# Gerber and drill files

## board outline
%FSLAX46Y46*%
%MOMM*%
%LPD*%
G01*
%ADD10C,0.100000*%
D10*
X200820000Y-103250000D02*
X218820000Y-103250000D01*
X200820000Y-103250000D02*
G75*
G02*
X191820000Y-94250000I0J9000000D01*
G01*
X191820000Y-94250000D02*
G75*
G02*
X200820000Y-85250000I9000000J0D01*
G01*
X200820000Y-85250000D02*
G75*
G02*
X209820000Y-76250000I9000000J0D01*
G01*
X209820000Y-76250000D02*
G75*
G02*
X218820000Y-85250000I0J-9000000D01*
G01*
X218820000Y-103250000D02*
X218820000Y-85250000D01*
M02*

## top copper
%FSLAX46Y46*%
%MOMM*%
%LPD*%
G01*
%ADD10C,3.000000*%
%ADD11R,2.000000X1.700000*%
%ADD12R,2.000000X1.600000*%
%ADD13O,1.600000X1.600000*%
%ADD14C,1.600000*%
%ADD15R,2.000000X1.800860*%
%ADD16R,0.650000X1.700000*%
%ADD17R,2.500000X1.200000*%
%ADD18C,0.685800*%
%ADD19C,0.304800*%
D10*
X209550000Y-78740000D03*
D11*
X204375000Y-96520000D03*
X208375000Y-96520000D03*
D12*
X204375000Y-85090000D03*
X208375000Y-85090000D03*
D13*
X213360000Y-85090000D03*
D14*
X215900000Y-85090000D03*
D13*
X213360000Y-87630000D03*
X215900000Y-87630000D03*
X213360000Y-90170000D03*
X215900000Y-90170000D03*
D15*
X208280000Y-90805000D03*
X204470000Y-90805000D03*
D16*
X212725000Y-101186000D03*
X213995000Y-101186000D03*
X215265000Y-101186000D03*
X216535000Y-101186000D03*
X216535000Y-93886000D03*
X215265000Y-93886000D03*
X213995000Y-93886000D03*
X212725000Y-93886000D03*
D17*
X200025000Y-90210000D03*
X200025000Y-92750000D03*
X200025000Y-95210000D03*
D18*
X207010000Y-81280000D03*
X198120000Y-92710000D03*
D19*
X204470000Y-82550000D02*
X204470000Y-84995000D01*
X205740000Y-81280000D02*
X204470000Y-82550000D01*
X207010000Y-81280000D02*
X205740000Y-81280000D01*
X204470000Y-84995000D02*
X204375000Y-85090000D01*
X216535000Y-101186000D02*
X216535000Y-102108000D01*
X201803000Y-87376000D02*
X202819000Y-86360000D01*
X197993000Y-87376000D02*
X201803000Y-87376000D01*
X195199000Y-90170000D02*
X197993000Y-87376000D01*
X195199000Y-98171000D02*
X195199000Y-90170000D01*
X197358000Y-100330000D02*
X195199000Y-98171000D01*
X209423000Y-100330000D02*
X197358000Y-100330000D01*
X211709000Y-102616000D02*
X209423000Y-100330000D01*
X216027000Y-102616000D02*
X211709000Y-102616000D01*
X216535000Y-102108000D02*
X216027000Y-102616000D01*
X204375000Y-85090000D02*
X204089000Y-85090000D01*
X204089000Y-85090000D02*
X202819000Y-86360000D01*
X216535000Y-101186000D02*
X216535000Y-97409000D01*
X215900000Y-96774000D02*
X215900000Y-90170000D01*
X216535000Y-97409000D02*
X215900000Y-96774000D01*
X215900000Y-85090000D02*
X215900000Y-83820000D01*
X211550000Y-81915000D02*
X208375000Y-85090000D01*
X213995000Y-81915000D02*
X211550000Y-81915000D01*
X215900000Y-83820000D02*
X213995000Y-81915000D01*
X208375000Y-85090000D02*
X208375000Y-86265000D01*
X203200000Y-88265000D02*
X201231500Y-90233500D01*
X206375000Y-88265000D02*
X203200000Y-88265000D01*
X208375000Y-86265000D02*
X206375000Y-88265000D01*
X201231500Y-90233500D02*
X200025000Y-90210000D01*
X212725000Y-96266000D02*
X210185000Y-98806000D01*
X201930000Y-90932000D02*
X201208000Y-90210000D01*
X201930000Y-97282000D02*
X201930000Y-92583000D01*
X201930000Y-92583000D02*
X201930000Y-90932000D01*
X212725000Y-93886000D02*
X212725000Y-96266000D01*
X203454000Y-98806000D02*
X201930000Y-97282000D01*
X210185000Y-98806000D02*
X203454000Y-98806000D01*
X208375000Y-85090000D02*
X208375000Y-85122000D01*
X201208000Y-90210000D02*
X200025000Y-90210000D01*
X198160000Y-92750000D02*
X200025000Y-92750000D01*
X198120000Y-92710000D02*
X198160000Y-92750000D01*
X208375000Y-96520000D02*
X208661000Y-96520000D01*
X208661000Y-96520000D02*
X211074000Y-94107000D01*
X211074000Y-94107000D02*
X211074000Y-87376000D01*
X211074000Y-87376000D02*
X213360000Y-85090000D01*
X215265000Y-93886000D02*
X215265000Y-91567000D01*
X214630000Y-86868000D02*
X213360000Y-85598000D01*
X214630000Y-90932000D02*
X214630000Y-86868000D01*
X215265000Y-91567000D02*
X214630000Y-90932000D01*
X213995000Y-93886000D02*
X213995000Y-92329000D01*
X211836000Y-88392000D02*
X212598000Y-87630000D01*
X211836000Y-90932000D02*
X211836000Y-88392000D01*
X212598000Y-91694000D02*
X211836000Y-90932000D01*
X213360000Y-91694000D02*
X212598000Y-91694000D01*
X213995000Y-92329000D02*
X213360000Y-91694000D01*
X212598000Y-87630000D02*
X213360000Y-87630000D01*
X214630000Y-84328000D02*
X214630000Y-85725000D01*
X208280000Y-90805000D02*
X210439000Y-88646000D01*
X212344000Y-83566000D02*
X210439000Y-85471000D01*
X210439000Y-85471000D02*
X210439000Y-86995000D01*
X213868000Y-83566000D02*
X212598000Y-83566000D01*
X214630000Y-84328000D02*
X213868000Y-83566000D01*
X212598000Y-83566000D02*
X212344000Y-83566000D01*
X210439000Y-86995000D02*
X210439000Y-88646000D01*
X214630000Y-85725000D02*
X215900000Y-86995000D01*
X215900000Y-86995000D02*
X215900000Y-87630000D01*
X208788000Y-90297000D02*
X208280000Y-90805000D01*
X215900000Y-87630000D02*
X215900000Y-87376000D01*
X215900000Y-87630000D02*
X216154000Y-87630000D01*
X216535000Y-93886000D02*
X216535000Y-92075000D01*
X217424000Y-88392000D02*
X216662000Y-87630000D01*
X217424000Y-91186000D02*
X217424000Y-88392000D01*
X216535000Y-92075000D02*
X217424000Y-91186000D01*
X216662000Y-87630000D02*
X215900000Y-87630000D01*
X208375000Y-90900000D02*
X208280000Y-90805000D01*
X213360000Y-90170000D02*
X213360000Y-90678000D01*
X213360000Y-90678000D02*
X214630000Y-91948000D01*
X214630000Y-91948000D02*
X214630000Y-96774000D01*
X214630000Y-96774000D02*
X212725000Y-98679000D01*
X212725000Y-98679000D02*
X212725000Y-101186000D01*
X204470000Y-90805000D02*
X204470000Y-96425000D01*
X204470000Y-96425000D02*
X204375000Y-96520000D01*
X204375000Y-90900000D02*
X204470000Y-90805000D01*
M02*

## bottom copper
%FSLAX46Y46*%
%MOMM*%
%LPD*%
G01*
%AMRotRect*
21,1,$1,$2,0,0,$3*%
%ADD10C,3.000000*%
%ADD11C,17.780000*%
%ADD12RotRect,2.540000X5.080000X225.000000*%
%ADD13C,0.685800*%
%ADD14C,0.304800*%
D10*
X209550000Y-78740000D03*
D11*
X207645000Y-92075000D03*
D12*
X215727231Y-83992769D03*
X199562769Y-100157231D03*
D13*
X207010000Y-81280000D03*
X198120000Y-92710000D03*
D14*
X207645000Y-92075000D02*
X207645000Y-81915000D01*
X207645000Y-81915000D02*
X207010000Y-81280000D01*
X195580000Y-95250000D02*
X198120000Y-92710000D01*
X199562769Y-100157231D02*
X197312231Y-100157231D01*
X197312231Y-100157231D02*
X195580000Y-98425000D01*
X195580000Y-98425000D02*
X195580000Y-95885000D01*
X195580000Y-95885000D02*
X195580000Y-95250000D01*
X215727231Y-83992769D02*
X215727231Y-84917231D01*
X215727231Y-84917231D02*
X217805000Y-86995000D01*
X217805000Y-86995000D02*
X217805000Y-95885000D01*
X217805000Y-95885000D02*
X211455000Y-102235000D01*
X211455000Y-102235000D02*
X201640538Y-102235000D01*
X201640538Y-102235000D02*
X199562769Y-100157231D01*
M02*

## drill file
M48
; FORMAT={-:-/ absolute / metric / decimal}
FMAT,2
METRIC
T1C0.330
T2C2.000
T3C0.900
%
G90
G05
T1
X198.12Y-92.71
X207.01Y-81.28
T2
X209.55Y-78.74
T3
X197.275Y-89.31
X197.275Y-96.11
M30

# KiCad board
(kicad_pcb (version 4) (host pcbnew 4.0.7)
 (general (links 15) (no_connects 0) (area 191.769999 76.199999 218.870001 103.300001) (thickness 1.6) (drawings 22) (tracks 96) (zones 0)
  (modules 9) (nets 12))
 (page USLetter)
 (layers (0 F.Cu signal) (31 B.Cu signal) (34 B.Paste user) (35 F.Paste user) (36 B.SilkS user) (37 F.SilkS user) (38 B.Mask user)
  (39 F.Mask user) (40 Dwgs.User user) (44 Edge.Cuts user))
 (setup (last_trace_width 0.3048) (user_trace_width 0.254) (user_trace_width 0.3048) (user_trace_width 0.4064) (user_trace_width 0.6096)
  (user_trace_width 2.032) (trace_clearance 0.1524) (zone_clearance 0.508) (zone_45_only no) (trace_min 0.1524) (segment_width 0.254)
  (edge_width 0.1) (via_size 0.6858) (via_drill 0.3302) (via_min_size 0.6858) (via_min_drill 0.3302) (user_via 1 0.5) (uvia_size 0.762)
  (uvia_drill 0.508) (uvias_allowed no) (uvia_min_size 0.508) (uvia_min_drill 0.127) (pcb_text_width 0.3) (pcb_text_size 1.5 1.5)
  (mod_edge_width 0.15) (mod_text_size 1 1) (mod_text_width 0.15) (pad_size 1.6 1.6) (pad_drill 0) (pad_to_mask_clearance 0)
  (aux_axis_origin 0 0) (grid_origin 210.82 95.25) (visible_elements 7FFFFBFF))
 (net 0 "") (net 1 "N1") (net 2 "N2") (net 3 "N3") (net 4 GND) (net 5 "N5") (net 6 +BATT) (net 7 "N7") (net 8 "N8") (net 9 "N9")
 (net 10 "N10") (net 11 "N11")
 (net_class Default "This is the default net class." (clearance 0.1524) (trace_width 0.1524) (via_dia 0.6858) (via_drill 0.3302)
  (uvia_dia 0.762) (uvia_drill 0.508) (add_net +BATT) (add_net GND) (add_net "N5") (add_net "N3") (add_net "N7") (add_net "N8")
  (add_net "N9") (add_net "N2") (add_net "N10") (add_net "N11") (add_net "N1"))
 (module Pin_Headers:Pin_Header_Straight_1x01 (layer F.Cu) (at 209.55 78.74)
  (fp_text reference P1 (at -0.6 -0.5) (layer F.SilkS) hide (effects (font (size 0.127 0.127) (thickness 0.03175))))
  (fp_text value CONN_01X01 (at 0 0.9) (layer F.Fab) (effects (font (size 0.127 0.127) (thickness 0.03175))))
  (pad 1 thru_hole circle (at 0 0) (size 3 3) (drill 2) (layers *.Cu *.Mask) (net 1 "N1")))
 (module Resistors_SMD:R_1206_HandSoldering (layer F.Cu) (at 206.375 96.52)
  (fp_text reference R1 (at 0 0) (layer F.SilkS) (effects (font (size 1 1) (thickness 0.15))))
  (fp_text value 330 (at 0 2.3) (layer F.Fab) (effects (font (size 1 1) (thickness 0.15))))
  (pad 1 smd rect (at -2 0) (size 2 1.7) (layers F.Cu F.Paste F.Mask) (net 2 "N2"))
  (pad 2 smd rect (at 2 0) (size 2 1.7) (layers F.Cu F.Paste F.Mask) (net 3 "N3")))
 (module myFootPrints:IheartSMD (layer F.Cu) (at 203.835 100.33)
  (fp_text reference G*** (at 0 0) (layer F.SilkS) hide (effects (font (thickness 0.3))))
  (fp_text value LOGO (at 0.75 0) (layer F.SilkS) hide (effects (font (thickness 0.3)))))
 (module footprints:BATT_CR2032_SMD (layer B.Cu) (at 207.645 92.075 225)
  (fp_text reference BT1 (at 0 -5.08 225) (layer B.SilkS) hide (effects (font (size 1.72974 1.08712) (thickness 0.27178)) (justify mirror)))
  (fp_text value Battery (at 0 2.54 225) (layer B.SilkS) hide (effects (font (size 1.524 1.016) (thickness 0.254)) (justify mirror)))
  (pad 2 smd circle (at 0 0 225) (size 17.78 17.78) (layers B.Cu B.Paste B.Mask) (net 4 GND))
  (pad 1 smd rect (at -11.43 0 225) (size 2.54 5.08) (layers B.Cu B.Paste B.Mask) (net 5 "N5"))
  (pad 1 smd rect (at 11.43 0 225) (size 2.54 5.08) (layers B.Cu B.Paste B.Mask) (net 5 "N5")))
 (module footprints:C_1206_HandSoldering (layer F.Cu) (at 206.375 85.09)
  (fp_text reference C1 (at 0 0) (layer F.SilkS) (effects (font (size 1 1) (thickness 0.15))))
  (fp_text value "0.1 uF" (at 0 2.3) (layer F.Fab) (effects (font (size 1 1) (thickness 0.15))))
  (pad 1 smd rect (at -2 0) (size 2 1.6) (layers F.Cu F.Paste F.Mask) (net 4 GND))
  (pad 2 smd rect (at 2 0) (size 2 1.6) (layers F.Cu F.Paste F.Mask) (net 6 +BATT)))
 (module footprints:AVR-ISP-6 (layer F.Cu) (at 213.36 85.09)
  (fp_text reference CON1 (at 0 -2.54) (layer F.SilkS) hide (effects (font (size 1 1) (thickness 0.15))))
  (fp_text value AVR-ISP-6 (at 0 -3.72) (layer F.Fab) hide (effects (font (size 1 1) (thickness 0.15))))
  (pad 1 smd oval (at 0 0) (size 1.6 1.6) (layers F.Cu F.Paste F.Mask) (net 3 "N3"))
  (pad 2 smd circle (at 2.54 0) (size 1.6 1.6) (layers F.Cu F.Paste F.Mask) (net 6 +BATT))
  (pad 3 smd oval (at 0 2.54) (size 1.6 1.6) (layers F.Cu F.Paste F.Mask) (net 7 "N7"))
  (pad 4 smd oval (at 2.54 2.54) (size 1.6 1.6) (layers F.Cu F.Paste F.Mask) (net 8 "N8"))
  (pad 5 smd oval (at 0 5.08) (size 1.6 1.6) (layers F.Cu F.Paste F.Mask) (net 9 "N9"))
  (pad 6 smd oval (at 2.54 5.08) (size 1.6 1.6) (layers F.Cu F.Paste F.Mask) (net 4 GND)))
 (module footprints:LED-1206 (layer F.Cu) (at 206.375 90.805)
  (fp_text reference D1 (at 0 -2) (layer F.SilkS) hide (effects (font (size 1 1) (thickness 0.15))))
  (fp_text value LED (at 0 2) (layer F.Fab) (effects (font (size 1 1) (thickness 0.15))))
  (pad 2 smd rect (at 1.905 0 180) (size 2 1.80086) (layers F.Cu F.Paste F.Mask) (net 8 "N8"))
  (pad 1 smd rect (at -1.905 0 180) (size 2 1.80086) (layers F.Cu F.Paste F.Mask) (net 2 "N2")))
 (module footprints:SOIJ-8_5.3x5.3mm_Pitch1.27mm (layer F.Cu) (at 214.63 97.536 90)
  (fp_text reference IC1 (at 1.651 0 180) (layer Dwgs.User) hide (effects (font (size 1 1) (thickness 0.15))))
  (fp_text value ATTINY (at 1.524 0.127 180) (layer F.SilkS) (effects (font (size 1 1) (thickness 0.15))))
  (pad 1 smd rect (at -3.65 -1.905 90) (size 1.7 0.65) (layers F.Cu F.Paste F.Mask) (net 9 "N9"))
  (pad 2 smd rect (at -3.65 -0.635 90) (size 1.7 0.65) (layers F.Cu F.Paste F.Mask) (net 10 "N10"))
  (pad 3 smd rect (at -3.65 0.635 90) (size 1.7 0.65) (layers F.Cu F.Paste F.Mask) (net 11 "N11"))
  (pad 4 smd rect (at -3.65 1.905 90) (size 1.7 0.65) (layers F.Cu F.Paste F.Mask) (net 4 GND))
  (pad 5 smd rect (at 3.65 1.905 90) (size 1.7 0.65) (layers F.Cu F.Paste F.Mask) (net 8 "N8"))
  (pad 6 smd rect (at 3.65 0.635 90) (size 1.7 0.65) (layers F.Cu F.Paste F.Mask) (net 3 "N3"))
  (pad 7 smd rect (at 3.65 -0.635 90) (size 1.7 0.65) (layers F.Cu F.Paste F.Mask) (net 7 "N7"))
  (pad 8 smd rect (at 3.65 -1.905 90) (size 1.7 0.65) (layers F.Cu F.Paste F.Mask) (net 6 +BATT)))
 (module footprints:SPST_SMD (layer F.Cu) (at 200.025 92.71 270)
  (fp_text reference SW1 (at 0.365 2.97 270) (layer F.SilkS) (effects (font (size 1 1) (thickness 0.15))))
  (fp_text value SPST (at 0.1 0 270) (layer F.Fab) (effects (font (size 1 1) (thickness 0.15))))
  (pad "" np_thru_hole circle (at 3.4 2.75 270) (size 0.9 0.9) (drill 0.9) (layers *.Cu *.Mask))
  (pad 1 smd rect (at -2.5 0 270) (size 1.2 2.5) (layers F.Cu F.Paste F.Mask) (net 6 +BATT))
  (pad 2 smd rect (at 0.04 0 270) (size 1.2 2.5) (layers F.Cu F.Paste F.Mask) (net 5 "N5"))
  (pad 3 smd rect (at 2.5 0 270) (size 1.2 2.5) (layers F.Cu F.Paste F.Mask))
  (pad "" np_thru_hole circle (at -3.4 2.75 270) (size 0.9 0.9) (drill 0.9) (layers *.Cu *.Mask)))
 (gr_line (start 200.82 103.25) (end 218.82 103.25) (angle 90) (layer Edge.Cuts) (width 0.1))
 (gr_arc (start 200.82 94.25) (end 200.82 103.25) (angle 90) (layer Edge.Cuts) (width 0.1))
 (gr_arc (start 200.82 94.25) (end 191.82 94.25) (angle 90) (layer Edge.Cuts) (width 0.1))
 (gr_arc (start 209.82 85.25) (end 200.82 85.25) (angle 90) (layer Edge.Cuts) (width 0.1))
 (gr_arc (start 209.82 85.25) (end 209.82 76.25) (angle 90) (layer Edge.Cuts) (width 0.1))
 (gr_line (start 218.82 103.25) (end 218.82 85.25) (angle 90) (layer Edge.Cuts) (width 0.1))
 (segment (start 207.645 92.075) (end 207.645 81.915) (width 0.3048) (layer B.Cu) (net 4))
 (segment (start 204.47 82.55) (end 204.47 84.995) (width 0.3048) (layer F.Cu) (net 4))
 (segment (start 205.74 81.28) (end 204.47 82.55) (width 0.3048) (layer F.Cu) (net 4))
 (segment (start 207.01 81.28) (end 205.74 81.28) (width 0.3048) (layer F.Cu) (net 4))
 (via (at 207.01 81.28) (size 0.6858) (drill 0.3302) (layers F.Cu B.Cu) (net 4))
 (segment (start 207.645 81.915) (end 207.01 81.28) (width 0.3048) (layer B.Cu) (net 4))
 (segment (start 204.47 84.995) (end 204.375 85.09) (width 0.3048) (layer F.Cu) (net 4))
 (segment (start 216.535 101.186) (end 216.535 102.108) (width 0.3048) (layer F.Cu) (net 4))
 (segment (start 201.803 87.376) (end 202.819 86.36) (width 0.3048) (layer F.Cu) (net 4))
 (segment (start 197.993 87.376) (end 201.803 87.376) (width 0.3048) (layer F.Cu) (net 4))
 (segment (start 195.199 90.17) (end 197.993 87.376) (width 0.3048) (layer F.Cu) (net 4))
 (segment (start 195.199 98.171) (end 195.199 90.17) (width 0.3048) (layer F.Cu) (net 4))
 (segment (start 197.358 100.33) (end 195.199 98.171) (width 0.3048) (layer F.Cu) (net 4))
 (segment (start 209.423 100.33) (end 197.358 100.33) (width 0.3048) (layer F.Cu) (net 4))
 (segment (start 211.709 102.616) (end 209.423 100.33) (width 0.3048) (layer F.Cu) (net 4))
 (segment (start 216.027 102.616) (end 211.709 102.616) (width 0.3048) (layer F.Cu) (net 4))
 (segment (start 216.535 102.108) (end 216.027 102.616) (width 0.3048) (layer F.Cu) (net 4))
 (segment (start 204.375 85.09) (end 204.089 85.09) (width 0.3048) (layer F.Cu) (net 4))
 (segment (start 204.089 85.09) (end 202.819 86.36) (width 0.3048) (layer F.Cu) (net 4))
 (segment (start 216.535 101.186) (end 216.535 97.409) (width 0.3048) (layer F.Cu) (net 4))
 (segment (start 215.9 96.774) (end 215.9 90.17) (width 0.3048) (layer F.Cu) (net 4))
 (segment (start 216.535 97.409) (end 215.9 96.774) (width 0.3048) (layer F.Cu) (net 4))
 (segment (start 215.9 85.09) (end 215.9 83.82) (width 0.3048) (layer F.Cu) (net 6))
 (segment (start 211.55 81.915) (end 208.375 85.09) (width 0.3048) (layer F.Cu) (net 6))
 (segment (start 213.995 81.915) (end 211.55 81.915) (width 0.3048) (layer F.Cu) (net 6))
 (segment (start 215.9 83.82) (end 213.995 81.915) (width 0.3048) (layer F.Cu) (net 6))
 (segment (start 208.375 85.09) (end 208.375 86.265) (width 0.3048) (layer F.Cu) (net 6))
 (segment (start 203.2 88.265) (end 201.2315 90.2335) (width 0.3048) (layer F.Cu) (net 6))
 (segment (start 206.375 88.265) (end 203.2 88.265) (width 0.3048) (layer F.Cu) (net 6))
 (segment (start 208.375 86.265) (end 206.375 88.265) (width 0.3048) (layer F.Cu) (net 6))
 (segment (start 201.2315 90.2335) (end 200.025 90.21) (width 0.3048) (layer F.Cu) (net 6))
 (segment (start 212.725 96.266) (end 210.185 98.806) (width 0.3048) (layer F.Cu) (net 6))
 (segment (start 201.93 90.932) (end 201.208 90.21) (width 0.3048) (layer F.Cu) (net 6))
 (segment (start 201.93 97.282) (end 201.93 92.583) (width 0.3048) (layer F.Cu) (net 6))
 (segment (start 201.93 92.583) (end 201.93 90.932) (width 0.3048) (layer F.Cu) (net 6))
 (segment (start 212.725 93.886) (end 212.725 96.266) (width 0.3048) (layer F.Cu) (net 6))
 (segment (start 203.454 98.806) (end 201.93 97.282) (width 0.3048) (layer F.Cu) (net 6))
 (segment (start 210.185 98.806) (end 203.454 98.806) (width 0.3048) (layer F.Cu) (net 6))
 (segment (start 208.375 85.09) (end 208.375 85.122) (width 0.3048) (layer F.Cu) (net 6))
 (segment (start 201.208 90.21) (end 200.025 90.21) (width 0.3048) (layer F.Cu) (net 6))
 (segment (start 195.58 95.25) (end 198.12 92.71) (width 0.3048) (layer B.Cu) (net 5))
 (segment (start 198.16 92.75) (end 200.025 92.75) (width 0.3048) (layer F.Cu) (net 5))
 (via (at 198.12 92.71) (size 0.6858) (drill 0.3302) (layers F.Cu B.Cu) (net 5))
 (segment (start 198.12 92.71) (end 198.16 92.75) (width 0.3048) (layer F.Cu) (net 5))
 (segment (start 199.562769 100.157231) (end 197.312231 100.157231) (width 0.3048) (layer B.Cu) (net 5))
 (segment (start 197.312231 100.157231) (end 195.58 98.425) (width 0.3048) (layer B.Cu) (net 5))
 (segment (start 195.58 98.425) (end 195.58 95.885) (width 0.3048) (layer B.Cu) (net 5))
 (segment (start 195.58 95.885) (end 195.58 95.25) (width 0.3048) (layer B.Cu) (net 5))
 (segment (start 215.727231 83.992769) (end 215.727231 84.917231) (width 0.3048) (layer B.Cu) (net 5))
 (segment (start 215.727231 84.917231) (end 217.805 86.995) (width 0.3048) (layer B.Cu) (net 5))
 (segment (start 217.805 86.995) (end 217.805 95.885) (width 0.3048) (layer B.Cu) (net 5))
 (segment (start 217.805 95.885) (end 211.455 102.235) (width 0.3048) (layer B.Cu) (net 5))
 (segment (start 211.455 102.235) (end 201.640538 102.235) (width 0.3048) (layer B.Cu) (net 5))
 (segment (start 201.640538 102.235) (end 199.562769 100.157231) (width 0.3048) (layer B.Cu) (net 5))
 (segment (start 208.375 96.52) (end 208.661 96.52) (width 0.3048) (layer F.Cu) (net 3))
 (segment (start 208.661 96.52) (end 211.074 94.107) (width 0.3048) (layer F.Cu) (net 3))
 (segment (start 211.074 94.107) (end 211.074 87.376) (width 0.3048) (layer F.Cu) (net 3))
 (segment (start 211.074 87.376) (end 213.36 85.09) (width 0.3048) (layer F.Cu) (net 3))
 (segment (start 215.265 93.886) (end 215.265 91.567) (width 0.3048) (layer F.Cu) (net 3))
 (segment (start 214.63 86.868) (end 213.36 85.598) (width 0.3048) (layer F.Cu) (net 3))
 (segment (start 214.63 90.932) (end 214.63 86.868) (width 0.3048) (layer F.Cu) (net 3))
 (segment (start 215.265 91.567) (end 214.63 90.932) (width 0.3048) (layer F.Cu) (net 3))
 (segment (start 213.995 93.886) (end 213.995 92.329) (width 0.3048) (layer F.Cu) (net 7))
 (segment (start 211.836 88.392) (end 212.598 87.63) (width 0.3048) (layer F.Cu) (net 7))
 (segment (start 211.836 90.932) (end 211.836 88.392) (width 0.3048) (layer F.Cu) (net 7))
 (segment (start 212.598 91.694) (end 211.836 90.932) (width 0.3048) (layer F.Cu) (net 7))
 (segment (start 213.36 91.694) (end 212.598 91.694) (width 0.3048) (layer F.Cu) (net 7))
 (segment (start 213.995 92.329) (end 213.36 91.694) (width 0.3048) (layer F.Cu) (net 7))
 (segment (start 212.598 87.63) (end 213.36 87.63) (width 0.3048) (layer F.Cu) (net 7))
 (segment (start 214.63 84.328) (end 214.63 85.725) (width 0.3048) (layer F.Cu) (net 8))
 (segment (start 208.28 90.805) (end 210.439 88.646) (width 0.3048) (layer F.Cu) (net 8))
 (segment (start 212.344 83.566) (end 210.439 85.471) (width 0.3048) (layer F.Cu) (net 8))
 (segment (start 210.439 85.471) (end 210.439 86.995) (width 0.3048) (layer F.Cu) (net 8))
 (segment (start 213.868 83.566) (end 212.598 83.566) (width 0.3048) (layer F.Cu) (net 8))
 (segment (start 214.63 84.328) (end 213.868 83.566) (width 0.3048) (layer F.Cu) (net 8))
 (segment (start 212.598 83.566) (end 212.344 83.566) (width 0.3048) (layer F.Cu) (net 8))
 (segment (start 210.439 86.995) (end 210.439 88.646) (width 0.3048) (layer F.Cu) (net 8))
 (segment (start 214.63 85.725) (end 215.9 86.995) (width 0.3048) (layer F.Cu) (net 8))
 (segment (start 215.9 86.995) (end 215.9 87.63) (width 0.3048) (layer F.Cu) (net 8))
 (segment (start 208.788 90.297) (end 208.28 90.805) (width 0.3048) (layer F.Cu) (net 8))
 (segment (start 215.9 87.63) (end 215.9 87.376) (width 0.3048) (layer F.Cu) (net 8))
 (segment (start 215.9 87.63) (end 216.154 87.63) (width 0.3048) (layer F.Cu) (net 8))
 (segment (start 216.535 93.886) (end 216.535 92.075) (width 0.3048) (layer F.Cu) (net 8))
 (segment (start 217.424 88.392) (end 216.662 87.63) (width 0.3048) (layer F.Cu) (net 8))
 (segment (start 217.424 91.186) (end 217.424 88.392) (width 0.3048) (layer F.Cu) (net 8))
 (segment (start 216.535 92.075) (end 217.424 91.186) (width 0.3048) (layer F.Cu) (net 8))
 (segment (start 216.662 87.63) (end 215.9 87.63) (width 0.3048) (layer F.Cu) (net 8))
 (segment (start 208.375 90.9) (end 208.28 90.805) (width 0.3048) (layer F.Cu) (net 8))
 (segment (start 213.36 90.17) (end 213.36 90.678) (width 0.3048) (layer F.Cu) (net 9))
 (segment (start 213.36 90.678) (end 214.63 91.948) (width 0.3048) (layer F.Cu) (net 9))
 (segment (start 214.63 91.948) (end 214.63 96.774) (width 0.3048) (layer F.Cu) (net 9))
 (segment (start 214.63 96.774) (end 212.725 98.679) (width 0.3048) (layer F.Cu) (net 9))
 (segment (start 212.725 98.679) (end 212.725 101.186) (width 0.3048) (layer F.Cu) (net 9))
 (segment (start 204.47 90.805) (end 204.47 96.425) (width 0.3048) (layer F.Cu) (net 2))
 (segment (start 204.47 96.425) (end 204.375 96.52) (width 0.3048) (layer F.Cu) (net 2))
 (segment (start 204.375 90.9) (end 204.47 90.805) (width 0.3048) (layer F.Cu) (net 2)))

